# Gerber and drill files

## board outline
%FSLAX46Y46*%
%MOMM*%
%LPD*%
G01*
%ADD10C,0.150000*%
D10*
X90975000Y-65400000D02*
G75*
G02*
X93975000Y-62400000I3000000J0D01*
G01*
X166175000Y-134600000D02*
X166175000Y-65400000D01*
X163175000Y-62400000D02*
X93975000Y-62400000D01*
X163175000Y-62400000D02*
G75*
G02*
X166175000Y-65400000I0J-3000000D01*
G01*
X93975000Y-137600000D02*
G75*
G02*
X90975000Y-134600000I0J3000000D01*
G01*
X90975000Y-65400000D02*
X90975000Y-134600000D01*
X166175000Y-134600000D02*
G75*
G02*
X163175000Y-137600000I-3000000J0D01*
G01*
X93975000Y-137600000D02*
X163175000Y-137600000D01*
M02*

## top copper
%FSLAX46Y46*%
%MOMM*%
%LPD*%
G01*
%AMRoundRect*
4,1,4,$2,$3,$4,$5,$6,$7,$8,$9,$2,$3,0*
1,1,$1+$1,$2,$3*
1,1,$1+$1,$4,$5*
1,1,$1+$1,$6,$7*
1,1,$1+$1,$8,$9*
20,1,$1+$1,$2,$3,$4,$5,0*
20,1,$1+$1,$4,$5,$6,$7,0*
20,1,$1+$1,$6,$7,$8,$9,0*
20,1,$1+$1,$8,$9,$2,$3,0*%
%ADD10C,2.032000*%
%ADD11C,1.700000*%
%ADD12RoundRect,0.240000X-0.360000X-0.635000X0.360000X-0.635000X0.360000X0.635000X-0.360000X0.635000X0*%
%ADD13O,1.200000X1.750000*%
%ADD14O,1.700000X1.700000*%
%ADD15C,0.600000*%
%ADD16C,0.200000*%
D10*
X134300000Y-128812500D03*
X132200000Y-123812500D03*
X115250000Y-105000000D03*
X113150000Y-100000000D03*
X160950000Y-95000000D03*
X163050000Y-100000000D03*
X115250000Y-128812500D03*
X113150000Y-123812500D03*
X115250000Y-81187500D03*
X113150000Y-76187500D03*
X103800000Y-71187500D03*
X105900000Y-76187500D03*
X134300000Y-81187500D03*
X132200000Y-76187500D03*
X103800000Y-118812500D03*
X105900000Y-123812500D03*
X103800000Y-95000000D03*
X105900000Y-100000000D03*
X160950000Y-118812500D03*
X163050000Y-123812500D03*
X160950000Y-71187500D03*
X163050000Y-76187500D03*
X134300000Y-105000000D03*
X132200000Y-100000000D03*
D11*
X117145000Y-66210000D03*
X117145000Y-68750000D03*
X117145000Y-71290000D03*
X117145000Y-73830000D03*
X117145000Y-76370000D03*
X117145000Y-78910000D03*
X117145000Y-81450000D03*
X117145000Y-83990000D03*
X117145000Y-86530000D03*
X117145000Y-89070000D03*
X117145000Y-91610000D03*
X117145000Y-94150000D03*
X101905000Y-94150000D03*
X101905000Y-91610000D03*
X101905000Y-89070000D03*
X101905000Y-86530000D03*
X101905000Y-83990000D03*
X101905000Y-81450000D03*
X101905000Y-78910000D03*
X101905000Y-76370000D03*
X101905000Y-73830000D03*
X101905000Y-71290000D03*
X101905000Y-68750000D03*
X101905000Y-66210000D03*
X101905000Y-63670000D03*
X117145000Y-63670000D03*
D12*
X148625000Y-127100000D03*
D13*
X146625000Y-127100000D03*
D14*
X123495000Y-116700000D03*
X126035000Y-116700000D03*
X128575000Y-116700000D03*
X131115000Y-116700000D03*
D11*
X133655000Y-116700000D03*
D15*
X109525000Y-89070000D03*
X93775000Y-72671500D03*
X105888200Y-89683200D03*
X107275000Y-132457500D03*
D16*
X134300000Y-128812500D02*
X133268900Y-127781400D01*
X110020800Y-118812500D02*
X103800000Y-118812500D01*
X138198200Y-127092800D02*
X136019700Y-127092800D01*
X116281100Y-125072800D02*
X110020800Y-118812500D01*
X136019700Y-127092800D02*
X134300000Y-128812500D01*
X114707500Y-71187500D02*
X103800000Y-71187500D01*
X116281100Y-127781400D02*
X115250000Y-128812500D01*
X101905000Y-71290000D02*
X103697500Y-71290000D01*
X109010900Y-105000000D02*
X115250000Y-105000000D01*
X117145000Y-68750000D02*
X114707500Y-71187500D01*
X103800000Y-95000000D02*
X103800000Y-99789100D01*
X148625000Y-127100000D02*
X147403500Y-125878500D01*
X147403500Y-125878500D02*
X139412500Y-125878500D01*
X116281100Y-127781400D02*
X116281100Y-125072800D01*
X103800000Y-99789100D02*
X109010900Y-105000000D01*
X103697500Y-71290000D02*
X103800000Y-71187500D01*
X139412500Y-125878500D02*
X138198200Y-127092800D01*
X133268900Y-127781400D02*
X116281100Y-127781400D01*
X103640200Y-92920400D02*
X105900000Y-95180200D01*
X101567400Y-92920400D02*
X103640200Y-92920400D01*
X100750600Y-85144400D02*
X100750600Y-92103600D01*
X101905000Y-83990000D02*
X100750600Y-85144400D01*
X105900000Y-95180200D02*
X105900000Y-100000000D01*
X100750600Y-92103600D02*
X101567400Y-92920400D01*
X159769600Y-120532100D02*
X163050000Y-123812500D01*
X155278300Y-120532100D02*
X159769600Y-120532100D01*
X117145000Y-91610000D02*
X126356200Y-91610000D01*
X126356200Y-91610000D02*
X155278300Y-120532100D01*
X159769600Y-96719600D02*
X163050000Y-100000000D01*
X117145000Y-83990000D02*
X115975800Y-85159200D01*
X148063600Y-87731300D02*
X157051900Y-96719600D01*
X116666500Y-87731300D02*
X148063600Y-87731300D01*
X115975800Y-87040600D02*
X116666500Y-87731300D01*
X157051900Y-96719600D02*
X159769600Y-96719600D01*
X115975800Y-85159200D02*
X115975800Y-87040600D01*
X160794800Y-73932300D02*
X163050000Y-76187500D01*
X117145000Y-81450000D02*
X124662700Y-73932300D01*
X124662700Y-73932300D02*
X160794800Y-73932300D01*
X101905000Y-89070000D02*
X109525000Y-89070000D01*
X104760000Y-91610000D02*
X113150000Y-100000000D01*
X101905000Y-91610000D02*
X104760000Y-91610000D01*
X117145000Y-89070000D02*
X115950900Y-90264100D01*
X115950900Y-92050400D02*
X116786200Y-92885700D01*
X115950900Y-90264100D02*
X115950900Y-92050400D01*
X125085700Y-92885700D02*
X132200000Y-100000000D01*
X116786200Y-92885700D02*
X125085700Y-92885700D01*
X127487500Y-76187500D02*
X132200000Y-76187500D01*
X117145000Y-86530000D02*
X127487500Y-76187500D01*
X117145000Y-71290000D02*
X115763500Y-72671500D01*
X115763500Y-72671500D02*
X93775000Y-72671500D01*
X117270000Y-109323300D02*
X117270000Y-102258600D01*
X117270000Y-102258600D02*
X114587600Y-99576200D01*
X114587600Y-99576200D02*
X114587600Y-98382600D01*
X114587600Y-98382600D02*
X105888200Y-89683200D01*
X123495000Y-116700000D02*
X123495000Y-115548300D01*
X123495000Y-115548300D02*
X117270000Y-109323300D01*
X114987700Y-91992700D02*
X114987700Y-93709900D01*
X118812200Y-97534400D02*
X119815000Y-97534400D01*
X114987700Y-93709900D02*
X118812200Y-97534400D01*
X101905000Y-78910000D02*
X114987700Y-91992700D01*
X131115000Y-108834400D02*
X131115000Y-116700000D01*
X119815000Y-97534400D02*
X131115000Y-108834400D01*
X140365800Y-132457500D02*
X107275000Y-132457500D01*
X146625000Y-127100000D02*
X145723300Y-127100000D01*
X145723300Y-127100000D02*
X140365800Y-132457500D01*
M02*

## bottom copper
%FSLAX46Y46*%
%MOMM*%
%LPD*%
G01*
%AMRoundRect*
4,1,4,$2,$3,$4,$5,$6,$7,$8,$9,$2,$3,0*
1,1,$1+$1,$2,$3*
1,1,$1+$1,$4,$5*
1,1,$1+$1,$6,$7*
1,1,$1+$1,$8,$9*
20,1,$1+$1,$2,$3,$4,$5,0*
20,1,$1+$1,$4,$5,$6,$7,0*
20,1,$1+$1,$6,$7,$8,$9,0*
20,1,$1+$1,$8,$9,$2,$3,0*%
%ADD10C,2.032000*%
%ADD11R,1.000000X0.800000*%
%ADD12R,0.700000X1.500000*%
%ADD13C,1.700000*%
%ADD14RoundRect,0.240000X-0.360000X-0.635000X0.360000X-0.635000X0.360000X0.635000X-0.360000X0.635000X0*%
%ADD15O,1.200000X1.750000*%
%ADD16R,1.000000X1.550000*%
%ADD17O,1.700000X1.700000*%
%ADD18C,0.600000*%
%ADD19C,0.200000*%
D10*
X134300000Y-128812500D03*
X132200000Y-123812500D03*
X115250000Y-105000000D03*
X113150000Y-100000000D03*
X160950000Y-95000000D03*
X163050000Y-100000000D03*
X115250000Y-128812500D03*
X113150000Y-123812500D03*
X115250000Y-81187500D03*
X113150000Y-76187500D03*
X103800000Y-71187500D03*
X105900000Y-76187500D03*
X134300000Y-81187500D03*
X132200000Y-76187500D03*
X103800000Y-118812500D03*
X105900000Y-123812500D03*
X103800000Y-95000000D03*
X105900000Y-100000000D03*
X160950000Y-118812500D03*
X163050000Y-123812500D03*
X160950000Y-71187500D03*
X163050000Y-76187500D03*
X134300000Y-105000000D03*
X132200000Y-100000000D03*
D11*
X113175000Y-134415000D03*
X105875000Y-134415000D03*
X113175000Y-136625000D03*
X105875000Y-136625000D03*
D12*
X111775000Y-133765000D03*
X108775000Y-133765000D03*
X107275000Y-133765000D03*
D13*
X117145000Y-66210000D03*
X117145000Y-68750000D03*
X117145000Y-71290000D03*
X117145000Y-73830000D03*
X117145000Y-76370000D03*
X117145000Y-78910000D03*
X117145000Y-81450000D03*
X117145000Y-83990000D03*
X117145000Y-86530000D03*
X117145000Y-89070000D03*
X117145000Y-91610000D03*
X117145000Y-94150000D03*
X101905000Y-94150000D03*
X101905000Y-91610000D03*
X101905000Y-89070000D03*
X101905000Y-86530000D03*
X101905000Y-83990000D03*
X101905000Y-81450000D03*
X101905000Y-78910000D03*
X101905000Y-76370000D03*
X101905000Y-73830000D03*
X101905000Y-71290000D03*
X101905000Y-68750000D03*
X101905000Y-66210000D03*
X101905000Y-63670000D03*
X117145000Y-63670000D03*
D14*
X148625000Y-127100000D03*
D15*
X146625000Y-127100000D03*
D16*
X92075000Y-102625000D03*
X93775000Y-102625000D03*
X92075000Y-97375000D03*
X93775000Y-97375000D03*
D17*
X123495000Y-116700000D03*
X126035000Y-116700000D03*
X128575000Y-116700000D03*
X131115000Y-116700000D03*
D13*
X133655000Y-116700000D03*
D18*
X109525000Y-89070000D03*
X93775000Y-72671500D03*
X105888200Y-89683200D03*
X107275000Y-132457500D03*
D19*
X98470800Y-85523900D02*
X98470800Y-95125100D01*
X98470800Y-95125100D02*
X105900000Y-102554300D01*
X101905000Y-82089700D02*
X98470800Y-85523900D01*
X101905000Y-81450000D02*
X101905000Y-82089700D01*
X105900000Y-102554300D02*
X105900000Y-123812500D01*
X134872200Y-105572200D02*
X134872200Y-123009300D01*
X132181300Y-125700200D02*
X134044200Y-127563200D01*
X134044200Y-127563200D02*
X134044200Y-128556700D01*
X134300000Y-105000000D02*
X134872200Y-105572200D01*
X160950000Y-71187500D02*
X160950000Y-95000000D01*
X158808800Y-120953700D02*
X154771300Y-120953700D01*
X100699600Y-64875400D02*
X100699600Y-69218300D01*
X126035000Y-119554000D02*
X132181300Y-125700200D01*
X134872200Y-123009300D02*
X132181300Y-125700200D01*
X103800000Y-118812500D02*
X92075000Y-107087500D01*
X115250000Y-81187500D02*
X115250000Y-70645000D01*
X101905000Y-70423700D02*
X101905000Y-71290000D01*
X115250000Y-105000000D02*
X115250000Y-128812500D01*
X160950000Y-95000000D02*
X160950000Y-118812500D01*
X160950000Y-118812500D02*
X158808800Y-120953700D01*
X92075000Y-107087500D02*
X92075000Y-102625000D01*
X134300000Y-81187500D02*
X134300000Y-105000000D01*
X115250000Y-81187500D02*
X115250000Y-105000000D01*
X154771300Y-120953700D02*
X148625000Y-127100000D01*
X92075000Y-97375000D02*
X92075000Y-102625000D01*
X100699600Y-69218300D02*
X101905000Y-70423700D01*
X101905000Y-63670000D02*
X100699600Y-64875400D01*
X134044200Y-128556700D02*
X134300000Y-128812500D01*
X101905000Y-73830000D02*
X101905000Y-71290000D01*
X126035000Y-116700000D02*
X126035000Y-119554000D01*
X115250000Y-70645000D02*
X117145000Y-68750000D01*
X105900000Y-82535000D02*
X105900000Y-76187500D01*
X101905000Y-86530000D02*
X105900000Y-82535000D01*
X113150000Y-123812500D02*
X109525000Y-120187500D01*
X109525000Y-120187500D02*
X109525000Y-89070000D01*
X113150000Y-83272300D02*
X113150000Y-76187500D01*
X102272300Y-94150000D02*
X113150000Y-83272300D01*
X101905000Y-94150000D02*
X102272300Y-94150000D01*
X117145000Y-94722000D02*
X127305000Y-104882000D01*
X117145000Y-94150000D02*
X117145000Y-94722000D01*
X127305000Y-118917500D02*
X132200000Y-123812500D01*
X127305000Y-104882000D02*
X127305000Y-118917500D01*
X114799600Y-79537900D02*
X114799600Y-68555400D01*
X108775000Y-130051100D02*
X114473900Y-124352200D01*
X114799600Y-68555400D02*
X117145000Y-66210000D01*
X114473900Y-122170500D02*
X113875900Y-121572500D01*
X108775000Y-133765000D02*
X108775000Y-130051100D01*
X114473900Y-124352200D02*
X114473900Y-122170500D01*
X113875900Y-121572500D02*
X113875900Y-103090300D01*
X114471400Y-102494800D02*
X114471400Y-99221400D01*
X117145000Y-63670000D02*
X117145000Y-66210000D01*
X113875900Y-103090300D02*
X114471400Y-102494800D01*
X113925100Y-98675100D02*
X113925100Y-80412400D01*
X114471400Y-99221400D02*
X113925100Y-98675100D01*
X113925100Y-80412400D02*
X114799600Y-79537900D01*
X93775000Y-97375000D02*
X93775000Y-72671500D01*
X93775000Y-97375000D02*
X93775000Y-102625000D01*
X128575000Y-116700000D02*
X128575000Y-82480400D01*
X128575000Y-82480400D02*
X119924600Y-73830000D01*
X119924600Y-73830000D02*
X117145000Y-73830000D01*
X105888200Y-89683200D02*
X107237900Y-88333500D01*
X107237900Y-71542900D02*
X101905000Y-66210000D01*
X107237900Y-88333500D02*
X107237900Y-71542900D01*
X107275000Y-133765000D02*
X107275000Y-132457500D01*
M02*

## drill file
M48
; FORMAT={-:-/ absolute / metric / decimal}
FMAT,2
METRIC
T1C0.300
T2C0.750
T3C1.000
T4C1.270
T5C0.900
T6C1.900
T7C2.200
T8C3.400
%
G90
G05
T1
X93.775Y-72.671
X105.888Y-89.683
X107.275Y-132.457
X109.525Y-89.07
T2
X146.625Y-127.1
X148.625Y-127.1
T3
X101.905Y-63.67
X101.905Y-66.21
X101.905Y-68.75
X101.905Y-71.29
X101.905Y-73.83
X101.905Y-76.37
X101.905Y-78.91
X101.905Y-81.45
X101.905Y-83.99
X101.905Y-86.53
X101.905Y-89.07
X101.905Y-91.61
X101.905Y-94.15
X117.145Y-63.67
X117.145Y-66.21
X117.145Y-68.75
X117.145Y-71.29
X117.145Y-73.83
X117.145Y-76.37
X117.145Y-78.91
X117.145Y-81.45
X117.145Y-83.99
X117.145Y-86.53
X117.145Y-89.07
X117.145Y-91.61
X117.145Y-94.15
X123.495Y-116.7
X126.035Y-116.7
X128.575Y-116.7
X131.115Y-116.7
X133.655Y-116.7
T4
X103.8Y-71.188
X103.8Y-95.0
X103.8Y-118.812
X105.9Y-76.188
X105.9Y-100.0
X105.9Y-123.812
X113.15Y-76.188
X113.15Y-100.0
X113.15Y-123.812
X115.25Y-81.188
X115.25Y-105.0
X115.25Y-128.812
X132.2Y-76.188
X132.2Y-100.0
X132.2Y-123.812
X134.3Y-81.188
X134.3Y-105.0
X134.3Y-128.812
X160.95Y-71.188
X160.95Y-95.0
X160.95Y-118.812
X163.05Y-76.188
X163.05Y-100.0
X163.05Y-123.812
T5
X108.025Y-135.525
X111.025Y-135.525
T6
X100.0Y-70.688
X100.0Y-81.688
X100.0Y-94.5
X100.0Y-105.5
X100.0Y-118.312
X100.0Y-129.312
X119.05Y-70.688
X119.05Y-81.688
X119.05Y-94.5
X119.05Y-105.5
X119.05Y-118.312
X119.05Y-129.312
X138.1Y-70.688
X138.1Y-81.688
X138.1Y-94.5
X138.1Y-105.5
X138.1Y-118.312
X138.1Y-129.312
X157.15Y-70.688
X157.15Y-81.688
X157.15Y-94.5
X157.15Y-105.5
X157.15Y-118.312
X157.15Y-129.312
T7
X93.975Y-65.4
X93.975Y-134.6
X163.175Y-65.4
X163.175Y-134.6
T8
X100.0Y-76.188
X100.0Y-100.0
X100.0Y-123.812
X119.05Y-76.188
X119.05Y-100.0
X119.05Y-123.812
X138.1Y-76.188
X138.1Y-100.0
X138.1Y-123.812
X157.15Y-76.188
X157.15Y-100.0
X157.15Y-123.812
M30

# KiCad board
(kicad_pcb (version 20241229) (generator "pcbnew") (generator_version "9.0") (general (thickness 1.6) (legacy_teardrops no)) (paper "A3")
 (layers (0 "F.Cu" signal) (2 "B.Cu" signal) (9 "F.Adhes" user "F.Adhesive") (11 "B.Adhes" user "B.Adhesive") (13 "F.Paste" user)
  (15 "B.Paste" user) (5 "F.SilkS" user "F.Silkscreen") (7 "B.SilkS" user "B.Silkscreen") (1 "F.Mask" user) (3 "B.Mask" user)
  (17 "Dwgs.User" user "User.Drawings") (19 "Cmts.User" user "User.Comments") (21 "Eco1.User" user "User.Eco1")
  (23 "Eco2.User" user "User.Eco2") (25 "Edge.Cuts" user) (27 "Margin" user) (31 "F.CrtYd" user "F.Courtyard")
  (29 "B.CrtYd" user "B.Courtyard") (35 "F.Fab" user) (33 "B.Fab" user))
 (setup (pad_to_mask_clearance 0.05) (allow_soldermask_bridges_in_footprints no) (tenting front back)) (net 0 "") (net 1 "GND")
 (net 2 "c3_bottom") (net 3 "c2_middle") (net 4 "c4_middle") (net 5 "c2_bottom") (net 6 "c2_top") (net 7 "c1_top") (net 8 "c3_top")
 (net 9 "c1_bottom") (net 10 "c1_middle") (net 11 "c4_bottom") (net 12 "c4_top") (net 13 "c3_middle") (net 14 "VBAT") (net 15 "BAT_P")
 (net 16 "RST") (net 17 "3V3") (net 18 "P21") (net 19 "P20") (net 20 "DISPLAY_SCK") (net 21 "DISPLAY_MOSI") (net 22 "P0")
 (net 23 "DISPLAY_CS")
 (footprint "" (layer "F.Cu") (at 128.574999 100)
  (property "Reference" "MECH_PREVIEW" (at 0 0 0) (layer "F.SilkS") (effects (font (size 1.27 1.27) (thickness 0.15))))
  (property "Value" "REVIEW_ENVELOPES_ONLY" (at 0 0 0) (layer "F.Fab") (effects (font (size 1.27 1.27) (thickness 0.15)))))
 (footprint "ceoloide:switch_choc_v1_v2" (layer "F.Cu") (at 138.1 123.8125 90)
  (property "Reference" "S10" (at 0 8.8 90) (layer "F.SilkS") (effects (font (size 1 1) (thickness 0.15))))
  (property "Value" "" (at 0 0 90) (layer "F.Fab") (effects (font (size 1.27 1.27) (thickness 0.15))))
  (pad "" np_thru_hole circle (at -5.5 0 90) (size 1.9 1.9) (drill 1.9) (layers "*.Cu" "*.Mask"))
  (pad "" np_thru_hole circle (at 0 0 90) (size 3.4 3.4) (drill 3.4) (layers "*.Cu" "*.Mask"))
  (pad "" np_thru_hole circle (at 5.5 0 90) (size 1.9 1.9) (drill 1.9) (layers "*.Cu" "*.Mask"))
  (pad "1" thru_hole circle (at -5 -3.8 285) (size 2.032 2.032) (drill 1.27) (layers "*.Cu" "*.Mask") (remove_unused_layers no)
   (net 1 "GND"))
  (pad "2" thru_hole circle (at 0 -5.9 285) (size 2.032 2.032) (drill 1.27) (layers "*.Cu" "*.Mask") (remove_unused_layers no)
   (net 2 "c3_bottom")))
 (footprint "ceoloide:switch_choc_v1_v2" (layer "F.Cu") (at 119.05 100 90)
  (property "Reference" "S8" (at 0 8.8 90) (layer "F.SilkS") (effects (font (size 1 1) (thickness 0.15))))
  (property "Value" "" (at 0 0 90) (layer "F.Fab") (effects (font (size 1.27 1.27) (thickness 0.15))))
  (pad "" np_thru_hole circle (at -5.5 0 90) (size 1.9 1.9) (drill 1.9) (layers "*.Cu" "*.Mask"))
  (pad "" np_thru_hole circle (at 0 0 90) (size 3.4 3.4) (drill 3.4) (layers "*.Cu" "*.Mask"))
  (pad "" np_thru_hole circle (at 5.5 0 90) (size 1.9 1.9) (drill 1.9) (layers "*.Cu" "*.Mask"))
  (pad "1" thru_hole circle (at -5 -3.8 285) (size 2.032 2.032) (drill 1.27) (layers "*.Cu" "*.Mask") (remove_unused_layers no)
   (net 1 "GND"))
  (pad "2" thru_hole circle (at 0 -5.9 285) (size 2.032 2.032) (drill 1.27) (layers "*.Cu" "*.Mask") (remove_unused_layers no)
   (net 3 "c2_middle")))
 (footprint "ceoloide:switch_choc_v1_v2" (layer "F.Cu") (at 157.15 100 -90)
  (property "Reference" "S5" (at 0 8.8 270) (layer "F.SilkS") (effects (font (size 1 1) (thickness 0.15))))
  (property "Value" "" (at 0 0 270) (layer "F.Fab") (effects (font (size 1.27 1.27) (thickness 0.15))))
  (pad "" np_thru_hole circle (at -5.5 0 270) (size 1.9 1.9) (drill 1.9) (layers "*.Cu" "*.Mask"))
  (pad "" np_thru_hole circle (at 0 0 270) (size 3.4 3.4) (drill 3.4) (layers "*.Cu" "*.Mask"))
  (pad "" np_thru_hole circle (at 5.5 0 270) (size 1.9 1.9) (drill 1.9) (layers "*.Cu" "*.Mask"))
  (pad "1" thru_hole circle (at -5 -3.8 105) (size 2.032 2.032) (drill 1.27) (layers "*.Cu" "*.Mask") (remove_unused_layers no)
   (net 1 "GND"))
  (pad "2" thru_hole circle (at 0 -5.9 105) (size 2.032 2.032) (drill 1.27) (layers "*.Cu" "*.Mask") (remove_unused_layers no)
   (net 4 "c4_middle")))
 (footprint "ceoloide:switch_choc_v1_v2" (layer "F.Cu") (at 119.05 123.8125 90)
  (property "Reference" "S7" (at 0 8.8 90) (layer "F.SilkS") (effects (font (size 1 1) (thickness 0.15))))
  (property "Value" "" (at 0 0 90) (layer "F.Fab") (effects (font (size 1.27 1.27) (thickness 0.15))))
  (pad "" np_thru_hole circle (at -5.5 0 90) (size 1.9 1.9) (drill 1.9) (layers "*.Cu" "*.Mask"))
  (pad "" np_thru_hole circle (at 0 0 90) (size 3.4 3.4) (drill 3.4) (layers "*.Cu" "*.Mask"))
  (pad "" np_thru_hole circle (at 5.5 0 90) (size 1.9 1.9) (drill 1.9) (layers "*.Cu" "*.Mask"))
  (pad "1" thru_hole circle (at -5 -3.8 285) (size 2.032 2.032) (drill 1.27) (layers "*.Cu" "*.Mask") (remove_unused_layers no)
   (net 1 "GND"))
  (pad "2" thru_hole circle (at 0 -5.9 285) (size 2.032 2.032) (drill 1.27) (layers "*.Cu" "*.Mask") (remove_unused_layers no)
   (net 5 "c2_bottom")))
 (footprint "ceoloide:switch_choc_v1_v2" (layer "F.Cu") (at 119.05 76.1875 90)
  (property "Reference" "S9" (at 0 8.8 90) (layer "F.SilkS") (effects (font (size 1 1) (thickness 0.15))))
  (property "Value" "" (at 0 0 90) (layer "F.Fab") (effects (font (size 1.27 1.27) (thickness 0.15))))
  (pad "" np_thru_hole circle (at -5.5 0 90) (size 1.9 1.9) (drill 1.9) (layers "*.Cu" "*.Mask"))
  (pad "" np_thru_hole circle (at 0 0 90) (size 3.4 3.4) (drill 3.4) (layers "*.Cu" "*.Mask"))
  (pad "" np_thru_hole circle (at 5.5 0 90) (size 1.9 1.9) (drill 1.9) (layers "*.Cu" "*.Mask"))
  (pad "1" thru_hole circle (at -5 -3.8 285) (size 2.032 2.032) (drill 1.27) (layers "*.Cu" "*.Mask") (remove_unused_layers no)
   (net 1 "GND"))
  (pad "2" thru_hole circle (at 0 -5.9 285) (size 2.032 2.032) (drill 1.27) (layers "*.Cu" "*.Mask") (remove_unused_layers no)
   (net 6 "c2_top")))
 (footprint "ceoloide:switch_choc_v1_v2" (layer "F.Cu") (at 100 76.1875 -90)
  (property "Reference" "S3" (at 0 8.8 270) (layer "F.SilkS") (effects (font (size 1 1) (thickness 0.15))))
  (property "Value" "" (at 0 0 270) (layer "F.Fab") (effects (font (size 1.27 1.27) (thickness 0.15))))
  (pad "" np_thru_hole circle (at -5.5 0 270) (size 1.9 1.9) (drill 1.9) (layers "*.Cu" "*.Mask"))
  (pad "" np_thru_hole circle (at 0 0 270) (size 3.4 3.4) (drill 3.4) (layers "*.Cu" "*.Mask"))
  (pad "" np_thru_hole circle (at 5.5 0 270) (size 1.9 1.9) (drill 1.9) (layers "*.Cu" "*.Mask"))
  (pad "1" thru_hole circle (at -5 -3.8 105) (size 2.032 2.032) (drill 1.27) (layers "*.Cu" "*.Mask") (remove_unused_layers no)
   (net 1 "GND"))
  (pad "2" thru_hole circle (at 0 -5.9 105) (size 2.032 2.032) (drill 1.27) (layers "*.Cu" "*.Mask") (remove_unused_layers no)
   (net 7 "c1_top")))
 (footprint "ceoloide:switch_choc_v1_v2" (layer "F.Cu") (at 138.1 76.1875 90)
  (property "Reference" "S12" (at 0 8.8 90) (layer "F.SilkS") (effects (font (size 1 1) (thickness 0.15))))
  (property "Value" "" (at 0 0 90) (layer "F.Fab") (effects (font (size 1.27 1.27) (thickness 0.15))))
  (pad "" np_thru_hole circle (at -5.5 0 90) (size 1.9 1.9) (drill 1.9) (layers "*.Cu" "*.Mask"))
  (pad "" np_thru_hole circle (at 0 0 90) (size 3.4 3.4) (drill 3.4) (layers "*.Cu" "*.Mask"))
  (pad "" np_thru_hole circle (at 5.5 0 90) (size 1.9 1.9) (drill 1.9) (layers "*.Cu" "*.Mask"))
  (pad "1" thru_hole circle (at -5 -3.8 285) (size 2.032 2.032) (drill 1.27) (layers "*.Cu" "*.Mask") (remove_unused_layers no)
   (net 1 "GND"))
  (pad "2" thru_hole circle (at 0 -5.9 285) (size 2.032 2.032) (drill 1.27) (layers "*.Cu" "*.Mask") (remove_unused_layers no)
   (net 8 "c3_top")))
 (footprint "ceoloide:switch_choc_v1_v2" (layer "F.Cu") (at 100 123.8125 -90)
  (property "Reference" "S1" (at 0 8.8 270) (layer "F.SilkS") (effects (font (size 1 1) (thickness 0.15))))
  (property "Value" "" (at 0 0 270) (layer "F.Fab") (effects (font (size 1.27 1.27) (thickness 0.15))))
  (pad "" np_thru_hole circle (at -5.5 0 270) (size 1.9 1.9) (drill 1.9) (layers "*.Cu" "*.Mask"))
  (pad "" np_thru_hole circle (at 0 0 270) (size 3.4 3.4) (drill 3.4) (layers "*.Cu" "*.Mask"))
  (pad "" np_thru_hole circle (at 5.5 0 270) (size 1.9 1.9) (drill 1.9) (layers "*.Cu" "*.Mask"))
  (pad "1" thru_hole circle (at -5 -3.8 105) (size 2.032 2.032) (drill 1.27) (layers "*.Cu" "*.Mask") (remove_unused_layers no)
   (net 1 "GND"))
  (pad "2" thru_hole circle (at 0 -5.9 105) (size 2.032 2.032) (drill 1.27) (layers "*.Cu" "*.Mask") (remove_unused_layers no)
   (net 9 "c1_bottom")))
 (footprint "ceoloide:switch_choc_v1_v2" (layer "F.Cu") (at 100 100 -90)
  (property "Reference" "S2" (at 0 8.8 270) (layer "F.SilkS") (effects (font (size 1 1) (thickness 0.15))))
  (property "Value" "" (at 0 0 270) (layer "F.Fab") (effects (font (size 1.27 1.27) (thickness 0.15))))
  (pad "" np_thru_hole circle (at -5.5 0 270) (size 1.9 1.9) (drill 1.9) (layers "*.Cu" "*.Mask"))
  (pad "" np_thru_hole circle (at 0 0 270) (size 3.4 3.4) (drill 3.4) (layers "*.Cu" "*.Mask"))
  (pad "" np_thru_hole circle (at 5.5 0 270) (size 1.9 1.9) (drill 1.9) (layers "*.Cu" "*.Mask"))
  (pad "1" thru_hole circle (at -5 -3.8 105) (size 2.032 2.032) (drill 1.27) (layers "*.Cu" "*.Mask") (remove_unused_layers no)
   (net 1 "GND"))
  (pad "2" thru_hole circle (at 0 -5.9 105) (size 2.032 2.032) (drill 1.27) (layers "*.Cu" "*.Mask") (remove_unused_layers no)
   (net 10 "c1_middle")))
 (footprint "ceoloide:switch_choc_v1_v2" (layer "F.Cu") (at 157.15 123.8125 -90)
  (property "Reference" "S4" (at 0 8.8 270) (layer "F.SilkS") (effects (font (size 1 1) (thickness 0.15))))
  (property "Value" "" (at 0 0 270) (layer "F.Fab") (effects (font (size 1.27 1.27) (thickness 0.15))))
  (pad "" np_thru_hole circle (at -5.5 0 270) (size 1.9 1.9) (drill 1.9) (layers "*.Cu" "*.Mask"))
  (pad "" np_thru_hole circle (at 0 0 270) (size 3.4 3.4) (drill 3.4) (layers "*.Cu" "*.Mask"))
  (pad "" np_thru_hole circle (at 5.5 0 270) (size 1.9 1.9) (drill 1.9) (layers "*.Cu" "*.Mask"))
  (pad "1" thru_hole circle (at -5 -3.8 105) (size 2.032 2.032) (drill 1.27) (layers "*.Cu" "*.Mask") (remove_unused_layers no)
   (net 1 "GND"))
  (pad "2" thru_hole circle (at 0 -5.9 105) (size 2.032 2.032) (drill 1.27) (layers "*.Cu" "*.Mask") (remove_unused_layers no)
   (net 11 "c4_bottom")))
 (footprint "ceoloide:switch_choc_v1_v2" (layer "F.Cu") (at 157.15 76.1875 -90)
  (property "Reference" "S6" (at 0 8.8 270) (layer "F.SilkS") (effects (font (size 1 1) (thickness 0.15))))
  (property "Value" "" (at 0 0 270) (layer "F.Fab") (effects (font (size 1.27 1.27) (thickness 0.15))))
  (pad "" np_thru_hole circle (at -5.5 0 270) (size 1.9 1.9) (drill 1.9) (layers "*.Cu" "*.Mask"))
  (pad "" np_thru_hole circle (at 0 0 270) (size 3.4 3.4) (drill 3.4) (layers "*.Cu" "*.Mask"))
  (pad "" np_thru_hole circle (at 5.5 0 270) (size 1.9 1.9) (drill 1.9) (layers "*.Cu" "*.Mask"))
  (pad "1" thru_hole circle (at -5 -3.8 105) (size 2.032 2.032) (drill 1.27) (layers "*.Cu" "*.Mask") (remove_unused_layers no)
   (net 1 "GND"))
  (pad "2" thru_hole circle (at 0 -5.9 105) (size 2.032 2.032) (drill 1.27) (layers "*.Cu" "*.Mask") (remove_unused_layers no)
   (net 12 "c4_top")))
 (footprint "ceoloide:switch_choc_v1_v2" (layer "F.Cu") (at 138.1 100 90)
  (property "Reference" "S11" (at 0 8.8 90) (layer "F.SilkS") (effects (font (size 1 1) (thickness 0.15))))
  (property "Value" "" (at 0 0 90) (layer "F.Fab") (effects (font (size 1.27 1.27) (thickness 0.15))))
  (pad "" np_thru_hole circle (at -5.5 0 90) (size 1.9 1.9) (drill 1.9) (layers "*.Cu" "*.Mask"))
  (pad "" np_thru_hole circle (at 0 0 90) (size 3.4 3.4) (drill 3.4) (layers "*.Cu" "*.Mask"))
  (pad "" np_thru_hole circle (at 5.5 0 90) (size 1.9 1.9) (drill 1.9) (layers "*.Cu" "*.Mask"))
  (pad "1" thru_hole circle (at -5 -3.8 285) (size 2.032 2.032) (drill 1.27) (layers "*.Cu" "*.Mask") (remove_unused_layers no)
   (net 1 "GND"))
  (pad "2" thru_hole circle (at 0 -5.9 285) (size 2.032 2.032) (drill 1.27) (layers "*.Cu" "*.Mask") (remove_unused_layers no)
   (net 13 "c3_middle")))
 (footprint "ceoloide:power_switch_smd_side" (layer "B.Cu") (at 109.525 135.5 -90)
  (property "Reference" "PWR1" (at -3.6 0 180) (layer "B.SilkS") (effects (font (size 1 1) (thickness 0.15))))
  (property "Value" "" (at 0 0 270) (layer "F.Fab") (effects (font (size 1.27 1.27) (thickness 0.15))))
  (pad "" smd rect (at -1.085 -3.65 180) (size 1 0.8) (layers "B.Cu" "B.Mask" "B.Paste"))
  (pad "" smd rect (at -1.085 3.65 180) (size 1 0.8) (layers "B.Cu" "B.Mask" "B.Paste"))
  (pad "" np_thru_hole circle (at 0.025 -1.5) (size 0.9 0.9) (drill 0.9) (layers "*.Cu" "*.Mask"))
  (pad "" np_thru_hole circle (at 0.025 1.5) (size 0.9 0.9) (drill 0.9) (layers "*.Cu" "*.Mask"))
  (pad "" smd rect (at 1.125 -3.65 180) (size 1 0.8) (layers "B.Cu" "B.Mask" "B.Paste"))
  (pad "" smd rect (at 1.125 3.65 180) (size 1 0.8) (layers "B.Cu" "B.Mask" "B.Paste"))
  (pad "1" smd rect (at -1.735 -2.25 180) (size 0.7 1.5) (layers "B.Cu" "B.Mask" "B.Paste"))
  (pad "2" smd rect (at -1.735 0.75 180) (size 0.7 1.5) (layers "B.Cu" "B.Mask" "B.Paste") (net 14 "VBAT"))
  (pad "3" smd rect (at -1.735 2.25 180) (size 0.7 1.5) (layers "B.Cu" "B.Mask" "B.Paste") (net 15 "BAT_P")))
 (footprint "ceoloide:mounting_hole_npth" (layer "B.Cu") (at 93.975 134.6)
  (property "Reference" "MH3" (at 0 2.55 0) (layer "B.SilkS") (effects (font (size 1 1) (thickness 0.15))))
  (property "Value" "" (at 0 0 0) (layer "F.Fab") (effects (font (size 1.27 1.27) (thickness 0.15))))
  (pad "" np_thru_hole circle (at 0 0) (size 2.2 2.2) (drill 2.2) (layers "*.Cu" "*.Mask")))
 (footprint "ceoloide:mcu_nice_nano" (layer "B.Cu") (at 109.525 78.91)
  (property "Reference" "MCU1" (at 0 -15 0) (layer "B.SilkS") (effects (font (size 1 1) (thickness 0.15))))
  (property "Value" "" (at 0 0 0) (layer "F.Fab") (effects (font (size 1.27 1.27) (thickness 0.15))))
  (pad "1" thru_hole circle (at 7.62 -12.7) (size 1.7 1.7) (drill 1) (layers "*.Cu" "*.Mask") (remove_unused_layers no) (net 14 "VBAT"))
  (pad "2" thru_hole circle (at 7.62 -10.16) (size 1.7 1.7) (drill 1) (layers "*.Cu" "*.Mask") (remove_unused_layers no) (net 1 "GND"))
  (pad "3" thru_hole circle (at 7.62 -7.62) (size 1.7 1.7) (drill 1) (layers "*.Cu" "*.Mask") (remove_unused_layers no) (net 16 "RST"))
  (pad "4" thru_hole circle (at 7.62 -5.08) (size 1.7 1.7) (drill 1) (layers "*.Cu" "*.Mask") (remove_unused_layers no) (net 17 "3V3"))
  (pad "5" thru_hole circle (at 7.62 -2.54) (size 1.7 1.7) (drill 1) (layers "*.Cu" "*.Mask") (remove_unused_layers no) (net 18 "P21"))
  (pad "6" thru_hole circle (at 7.62 0) (size 1.7 1.7) (drill 1) (layers "*.Cu" "*.Mask") (remove_unused_layers no) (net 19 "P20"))
  (pad "7" thru_hole circle (at 7.62 2.54) (size 1.7 1.7) (drill 1) (layers "*.Cu" "*.Mask") (remove_unused_layers no) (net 12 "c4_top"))
  (pad "8" thru_hole circle (at 7.62 5.08) (size 1.7 1.7) (drill 1) (layers "*.Cu" "*.Mask") (remove_unused_layers no) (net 4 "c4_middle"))
  (pad "9" thru_hole circle (at 7.62 7.62) (size 1.7 1.7) (drill 1) (layers "*.Cu" "*.Mask") (remove_unused_layers no) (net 8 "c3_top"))
  (pad "10" thru_hole circle (at 7.62 10.16) (size 1.7 1.7) (drill 1) (layers "*.Cu" "*.Mask") (remove_unused_layers no)
   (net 13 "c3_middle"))
  (pad "11" thru_hole circle (at 7.62 12.7) (size 1.7 1.7) (drill 1) (layers "*.Cu" "*.Mask") (remove_unused_layers no) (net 11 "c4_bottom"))
  (pad "12" thru_hole circle (at 7.62 15.24) (size 1.7 1.7) (drill 1) (layers "*.Cu" "*.Mask") (remove_unused_layers no) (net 2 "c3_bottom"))
  (pad "13" thru_hole circle (at -7.62 15.24) (size 1.7 1.7) (drill 1) (layers "*.Cu" "*.Mask") (remove_unused_layers no) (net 6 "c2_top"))
  (pad "14" thru_hole circle (at -7.62 12.7) (size 1.7 1.7) (drill 1) (layers "*.Cu" "*.Mask") (remove_unused_layers no) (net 3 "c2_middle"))
  (pad "15" thru_hole circle (at -7.62 10.16) (size 1.7 1.7) (drill 1) (layers "*.Cu" "*.Mask") (remove_unused_layers no)
   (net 5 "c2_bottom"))
  (pad "16" thru_hole circle (at -7.62 7.62) (size 1.7 1.7) (drill 1) (layers "*.Cu" "*.Mask") (remove_unused_layers no) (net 7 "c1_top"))
  (pad "17" thru_hole circle (at -7.62 5.08) (size 1.7 1.7) (drill 1) (layers "*.Cu" "*.Mask") (remove_unused_layers no)
   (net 10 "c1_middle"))
  (pad "18" thru_hole circle (at -7.62 2.54) (size 1.7 1.7) (drill 1) (layers "*.Cu" "*.Mask") (remove_unused_layers no) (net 9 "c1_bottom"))
  (pad "19" thru_hole circle (at -7.62 0) (size 1.7 1.7) (drill 1) (layers "*.Cu" "*.Mask") (remove_unused_layers no) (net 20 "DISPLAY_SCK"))
  (pad "20" thru_hole circle (at -7.62 -2.54) (size 1.7 1.7) (drill 1) (layers "*.Cu" "*.Mask") (remove_unused_layers no)
   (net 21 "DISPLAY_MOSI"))
  (pad "21" thru_hole circle (at -7.62 -5.08) (size 1.7 1.7) (drill 1) (layers "*.Cu" "*.Mask") (remove_unused_layers no) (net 1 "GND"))
  (pad "22" thru_hole circle (at -7.62 -7.62) (size 1.7 1.7) (drill 1) (layers "*.Cu" "*.Mask") (remove_unused_layers no) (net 1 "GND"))
  (pad "23" thru_hole circle (at -7.62 -10.16) (size 1.7 1.7) (drill 1) (layers "*.Cu" "*.Mask") (remove_unused_layers no) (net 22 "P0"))
  (pad "24" thru_hole circle (at -7.62 -12.7) (size 1.7 1.7) (drill 1) (layers "*.Cu" "*.Mask") (remove_unused_layers no)
   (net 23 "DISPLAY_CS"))
  (pad "25" thru_hole circle (at -7.62 -15.24) (size 1.7 1.7) (drill 1) (layers "*.Cu" "*.Mask") (remove_unused_layers no) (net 1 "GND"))
  (pad "26" thru_hole circle (at 7.62 -15.24) (size 1.7 1.7) (drill 1) (layers "*.Cu" "*.Mask") (remove_unused_layers no) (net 14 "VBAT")))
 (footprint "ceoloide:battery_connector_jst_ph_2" (layer "B.Cu") (at 147.625 127.1)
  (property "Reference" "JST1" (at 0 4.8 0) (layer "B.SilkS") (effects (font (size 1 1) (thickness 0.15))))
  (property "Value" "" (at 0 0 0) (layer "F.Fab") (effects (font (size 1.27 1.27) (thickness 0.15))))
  (pad "1" thru_hole roundrect (at 1 0) (size 1.2 1.75) (drill 0.75) (layers "*.Cu" "*.Mask") (remove_unused_layers no)
   (roundrect_rratio 0.2) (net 1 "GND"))
  (pad "2" thru_hole oval (at -1 0) (size 1.2 1.75) (drill 0.75) (layers "*.Cu" "*.Mask") (remove_unused_layers no) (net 15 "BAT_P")))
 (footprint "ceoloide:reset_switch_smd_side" (layer "B.Cu") (at 92.925 100 90)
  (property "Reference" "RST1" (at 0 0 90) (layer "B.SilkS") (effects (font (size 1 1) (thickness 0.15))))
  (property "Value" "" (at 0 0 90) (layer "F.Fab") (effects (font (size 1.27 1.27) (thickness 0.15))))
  (pad "1" smd rect (at -2.625 -0.85 270) (size 1.55 1) (layers "B.Cu" "B.Mask" "B.Paste") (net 1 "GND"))
  (pad "2" smd rect (at -2.625 0.85 270) (size 1.55 1) (layers "B.Cu" "B.Mask" "B.Paste") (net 16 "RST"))
  (pad "3" smd rect (at 2.625 -0.85 270) (size 1.55 1) (layers "B.Cu" "B.Mask" "B.Paste") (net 1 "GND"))
  (pad "4" smd rect (at 2.625 0.85 270) (size 1.55 1) (layers "B.Cu" "B.Mask" "B.Paste") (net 16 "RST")))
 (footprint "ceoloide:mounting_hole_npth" (layer "B.Cu") (at 163.175 65.4)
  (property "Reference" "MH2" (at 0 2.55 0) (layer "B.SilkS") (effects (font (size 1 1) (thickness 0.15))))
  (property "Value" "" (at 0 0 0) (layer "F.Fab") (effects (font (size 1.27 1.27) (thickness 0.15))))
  (pad "" np_thru_hole circle (at 0 0) (size 2.2 2.2) (drill 2.2) (layers "*.Cu" "*.Mask")))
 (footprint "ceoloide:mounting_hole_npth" (layer "B.Cu") (at 163.175 134.6)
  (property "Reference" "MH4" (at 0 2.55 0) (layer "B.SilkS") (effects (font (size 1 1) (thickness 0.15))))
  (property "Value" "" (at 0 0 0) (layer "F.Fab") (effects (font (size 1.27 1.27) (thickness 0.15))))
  (pad "" np_thru_hole circle (at 0 0) (size 2.2 2.2) (drill 2.2) (layers "*.Cu" "*.Mask")))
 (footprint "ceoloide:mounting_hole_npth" (layer "B.Cu") (at 93.975 65.4)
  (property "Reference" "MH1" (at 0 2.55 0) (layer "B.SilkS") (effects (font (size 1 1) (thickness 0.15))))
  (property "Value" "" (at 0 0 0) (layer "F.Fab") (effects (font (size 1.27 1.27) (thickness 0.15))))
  (pad "" np_thru_hole circle (at 0 0) (size 2.2 2.2) (drill 2.2) (layers "*.Cu" "*.Mask")))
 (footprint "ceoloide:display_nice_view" (layer "B.Cu") (at 128.575 100)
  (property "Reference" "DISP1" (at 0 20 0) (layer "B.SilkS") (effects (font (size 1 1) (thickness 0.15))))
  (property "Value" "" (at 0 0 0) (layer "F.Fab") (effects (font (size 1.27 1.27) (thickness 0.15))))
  (pad "1" thru_hole oval (at -5.08 16.7 270) (size 1.7 1.7) (drill 1) (layers "*.Cu" "*.Mask") (remove_unused_layers no)
   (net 23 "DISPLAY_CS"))
  (pad "2" thru_hole oval (at -2.54 16.7 270) (size 1.7 1.7) (drill 1) (layers "*.Cu" "*.Mask") (remove_unused_layers no) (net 1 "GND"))
  (pad "3" thru_hole oval (at 0 16.7 270) (size 1.7 1.7) (drill 1) (layers "*.Cu" "*.Mask") (remove_unused_layers no) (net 17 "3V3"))
  (pad "4" thru_hole oval (at 2.54 16.7 270) (size 1.7 1.7) (drill 1) (layers "*.Cu" "*.Mask") (remove_unused_layers no)
   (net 20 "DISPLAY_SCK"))
  (pad "5" thru_hole circle (at 5.08 16.7 270) (size 1.7 1.7) (drill 1) (layers "*.Cu" "*.Mask") (remove_unused_layers no)
   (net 21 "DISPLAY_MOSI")))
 (gr_arc (start 90.975 65.4) (mid 91.85368 63.27868) (end 93.975 62.4) (stroke (width 0.15) (type default)) (layer "Edge.Cuts"))
 (gr_line (start 166.175 134.6) (end 166.175 65.4) (stroke (width 0.15) (type default)) (layer "Edge.Cuts"))
 (gr_line (start 163.175 62.4) (end 93.975 62.4) (stroke (width 0.15) (type default)) (layer "Edge.Cuts"))
 (gr_arc (start 163.175 62.4) (mid 165.29632 63.27868) (end 166.175 65.4) (stroke (width 0.15) (type default)) (layer "Edge.Cuts"))
 (gr_arc (start 93.975 137.6) (mid 91.85368 136.72132) (end 90.975 134.6) (stroke (width 0.15) (type default)) (layer "Edge.Cuts"))
 (gr_line (start 90.975 65.4) (end 90.975 134.6) (stroke (width 0.15) (type default)) (layer "Edge.Cuts"))
 (gr_arc (start 166.175 134.6) (mid 165.29632 136.72132) (end 163.175 137.6) (stroke (width 0.15) (type default)) (layer "Edge.Cuts"))
 (gr_line (start 93.975 137.6) (end 163.175 137.6) (stroke (width 0.15) (type default)) (layer "Edge.Cuts"))
 (segment (start 98.4708 85.5239) (end 98.4708 95.1251) (width 0.2) (layer "B.Cu") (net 9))
 (segment (start 98.4708 95.1251) (end 105.9 102.5543) (width 0.2) (layer "B.Cu") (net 9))
 (segment (start 101.905 82.0897) (end 98.4708 85.5239) (width 0.2) (layer "B.Cu") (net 9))
 (segment (start 101.905 81.45) (end 101.905 82.0897) (width 0.2) (layer "B.Cu") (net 9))
 (segment (start 105.9 102.5543) (end 105.9 123.8125) (width 0.2) (layer "B.Cu") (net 9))
 (segment (start 134.3 128.8125) (end 133.2689 127.7814) (width 0.2) (layer "F.Cu") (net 1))
 (segment (start 110.0208 118.8125) (end 103.8 118.8125) (width 0.2) (layer "F.Cu") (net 1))
 (segment (start 138.1982 127.0928) (end 136.0197 127.0928) (width 0.2) (layer "F.Cu") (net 1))
 (segment (start 116.2811 125.0728) (end 110.0208 118.8125) (width 0.2) (layer "F.Cu") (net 1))
 (segment (start 136.0197 127.0928) (end 134.3 128.8125) (width 0.2) (layer "F.Cu") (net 1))
 (segment (start 114.7075 71.1875) (end 103.8 71.1875) (width 0.2) (layer "F.Cu") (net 1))
 (segment (start 116.2811 127.7814) (end 115.25 128.8125) (width 0.2) (layer "F.Cu") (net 1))
 (segment (start 101.905 71.29) (end 103.6975 71.29) (width 0.2) (layer "F.Cu") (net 1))
 (segment (start 109.0109 105) (end 115.25 105) (width 0.2) (layer "F.Cu") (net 1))
 (segment (start 117.145 68.75) (end 114.7075 71.1875) (width 0.2) (layer "F.Cu") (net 1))
 (segment (start 103.8 95) (end 103.8 99.7891) (width 0.2) (layer "F.Cu") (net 1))
 (segment (start 148.625 127.1) (end 147.4035 125.8785) (width 0.2) (layer "F.Cu") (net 1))
 (segment (start 147.4035 125.8785) (end 139.4125 125.8785) (width 0.2) (layer "F.Cu") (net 1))
 (segment (start 116.2811 127.7814) (end 116.2811 125.0728) (width 0.2) (layer "F.Cu") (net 1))
 (segment (start 103.8 99.7891) (end 109.0109 105) (width 0.2) (layer "F.Cu") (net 1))
 (segment (start 103.6975 71.29) (end 103.8 71.1875) (width 0.2) (layer "F.Cu") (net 1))
 (segment (start 139.4125 125.8785) (end 138.1982 127.0928) (width 0.2) (layer "F.Cu") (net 1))
 (segment (start 133.2689 127.7814) (end 116.2811 127.7814) (width 0.2) (layer "F.Cu") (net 1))
 (segment (start 134.8722 105.5722) (end 134.8722 123.0093) (width 0.2) (layer "B.Cu") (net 1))
 (segment (start 132.1813 125.7002) (end 134.0442 127.5632) (width 0.2) (layer "B.Cu") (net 1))
 (segment (start 134.0442 127.5632) (end 134.0442 128.5567) (width 0.2) (layer "B.Cu") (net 1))
 (segment (start 134.3 105) (end 134.8722 105.5722) (width 0.2) (layer "B.Cu") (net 1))
 (segment (start 160.95 71.1875) (end 160.95 95) (width 0.2) (layer "B.Cu") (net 1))
 (segment (start 158.8088 120.9537) (end 154.7713 120.9537) (width 0.2) (layer "B.Cu") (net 1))
 (segment (start 100.6996 64.8754) (end 100.6996 69.2183) (width 0.2) (layer "B.Cu") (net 1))
 (segment (start 126.035 119.554) (end 132.1813 125.7002) (width 0.2) (layer "B.Cu") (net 1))
 (segment (start 134.8722 123.0093) (end 132.1813 125.7002) (width 0.2) (layer "B.Cu") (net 1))
 (segment (start 103.8 118.8125) (end 92.075 107.0875) (width 0.2) (layer "B.Cu") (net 1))
 (segment (start 115.25 81.1875) (end 115.25 70.645) (width 0.2) (layer "B.Cu") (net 1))
 (segment (start 101.905 70.4237) (end 101.905 71.29) (width 0.2) (layer "B.Cu") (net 1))
 (segment (start 115.25 105) (end 115.25 128.8125) (width 0.2) (layer "B.Cu") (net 1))
 (segment (start 160.95 95) (end 160.95 118.8125) (width 0.2) (layer "B.Cu") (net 1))
 (segment (start 160.95 118.8125) (end 158.8088 120.9537) (width 0.2) (layer "B.Cu") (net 1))
 (segment (start 92.075 107.0875) (end 92.075 102.625) (width 0.2) (layer "B.Cu") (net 1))
 (segment (start 134.3 81.1875) (end 134.3 105) (width 0.2) (layer "B.Cu") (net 1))
 (segment (start 115.25 81.1875) (end 115.25 105) (width 0.2) (layer "B.Cu") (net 1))
 (segment (start 154.7713 120.9537) (end 148.625 127.1) (width 0.2) (layer "B.Cu") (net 1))
 (segment (start 92.075 97.375) (end 92.075 102.625) (width 0.2) (layer "B.Cu") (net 1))
 (segment (start 100.6996 69.2183) (end 101.905 70.4237) (width 0.2) (layer "B.Cu") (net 1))
 (segment (start 101.905 63.67) (end 100.6996 64.8754) (width 0.2) (layer "B.Cu") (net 1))
 (segment (start 134.0442 128.5567) (end 134.3 128.8125) (width 0.2) (layer "B.Cu") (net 1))
 (segment (start 101.905 73.83) (end 101.905 71.29) (width 0.2) (layer "B.Cu") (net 1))
 (segment (start 126.035 116.7) (end 126.035 119.554) (width 0.2) (layer "B.Cu") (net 1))
 (segment (start 115.25 70.645) (end 117.145 68.75) (width 0.2) (layer "B.Cu") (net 1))
 (segment (start 103.6402 92.9204) (end 105.9 95.1802) (width 0.2) (layer "F.Cu") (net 10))
 (segment (start 101.5674 92.9204) (end 103.6402 92.9204) (width 0.2) (layer "F.Cu") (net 10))
 (segment (start 100.7506 85.1444) (end 100.7506 92.1036) (width 0.2) (layer "F.Cu") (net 10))
 (segment (start 101.905 83.99) (end 100.7506 85.1444) (width 0.2) (layer "F.Cu") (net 10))
 (segment (start 105.9 95.1802) (end 105.9 100) (width 0.2) (layer "F.Cu") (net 10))
 (segment (start 100.7506 92.1036) (end 101.5674 92.9204) (width 0.2) (layer "F.Cu") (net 10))
 (segment (start 105.9 82.535) (end 105.9 76.1875) (width 0.2) (layer "B.Cu") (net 7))
 (segment (start 101.905 86.53) (end 105.9 82.535) (width 0.2) (layer "B.Cu") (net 7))
 (segment (start 159.7696 120.5321) (end 163.05 123.8125) (width 0.2) (layer "F.Cu") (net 11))
 (segment (start 155.2783 120.5321) (end 159.7696 120.5321) (width 0.2) (layer "F.Cu") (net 11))
 (segment (start 117.145 91.61) (end 126.3562 91.61) (width 0.2) (layer "F.Cu") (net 11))
 (segment (start 126.3562 91.61) (end 155.2783 120.5321) (width 0.2) (layer "F.Cu") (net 11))
 (segment (start 159.7696 96.7196) (end 163.05 100) (width 0.2) (layer "F.Cu") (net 4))
 (segment (start 117.145 83.99) (end 115.9758 85.1592) (width 0.2) (layer "F.Cu") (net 4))
 (segment (start 148.0636 87.7313) (end 157.0519 96.7196) (width 0.2) (layer "F.Cu") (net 4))
 (segment (start 116.6665 87.7313) (end 148.0636 87.7313) (width 0.2) (layer "F.Cu") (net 4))
 (segment (start 115.9758 87.0406) (end 116.6665 87.7313) (width 0.2) (layer "F.Cu") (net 4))
 (segment (start 157.0519 96.7196) (end 159.7696 96.7196) (width 0.2) (layer "F.Cu") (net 4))
 (segment (start 115.9758 85.1592) (end 115.9758 87.0406) (width 0.2) (layer "F.Cu") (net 4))
 (segment (start 160.7948 73.9323) (end 163.05 76.1875) (width 0.2) (layer "F.Cu") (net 12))
 (segment (start 117.145 81.45) (end 124.6627 73.9323) (width 0.2) (layer "F.Cu") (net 12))
 (segment (start 124.6627 73.9323) (end 160.7948 73.9323) (width 0.2) (layer "F.Cu") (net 12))
 (segment (start 101.905 89.07) (end 109.525 89.07) (width 0.2) (layer "F.Cu") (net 5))
 (via (at 109.525 89.07) (size 0.6) (drill 0.3) (layers "F.Cu" "B.Cu") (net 5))
 (segment (start 113.15 123.8125) (end 109.525 120.1875) (width 0.2) (layer "B.Cu") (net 5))
 (segment (start 109.525 120.1875) (end 109.525 89.07) (width 0.2) (layer "B.Cu") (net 5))
 (segment (start 104.76 91.61) (end 113.15 100) (width 0.2) (layer "F.Cu") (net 3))
 (segment (start 101.905 91.61) (end 104.76 91.61) (width 0.2) (layer "F.Cu") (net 3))
 (segment (start 113.15 83.2723) (end 113.15 76.1875) (width 0.2) (layer "B.Cu") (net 6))
 (segment (start 102.2723 94.15) (end 113.15 83.2723) (width 0.2) (layer "B.Cu") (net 6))
 (segment (start 101.905 94.15) (end 102.2723 94.15) (width 0.2) (layer "B.Cu") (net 6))
 (segment (start 117.145 94.722) (end 127.305 104.882) (width 0.2) (layer "B.Cu") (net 2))
 (segment (start 117.145 94.15) (end 117.145 94.722) (width 0.2) (layer "B.Cu") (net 2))
 (segment (start 127.305 118.9175) (end 132.2 123.8125) (width 0.2) (layer "B.Cu") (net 2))
 (segment (start 127.305 104.882) (end 127.305 118.9175) (width 0.2) (layer "B.Cu") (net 2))
 (segment (start 117.145 89.07) (end 115.9509 90.2641) (width 0.2) (layer "F.Cu") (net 13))
 (segment (start 115.9509 92.0504) (end 116.7862 92.8857) (width 0.2) (layer "F.Cu") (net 13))
 (segment (start 115.9509 90.2641) (end 115.9509 92.0504) (width 0.2) (layer "F.Cu") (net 13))
 (segment (start 125.0857 92.8857) (end 132.2 100) (width 0.2) (layer "F.Cu") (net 13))
 (segment (start 116.7862 92.8857) (end 125.0857 92.8857) (width 0.2) (layer "F.Cu") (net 13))
 (segment (start 127.4875 76.1875) (end 132.2 76.1875) (width 0.2) (layer "F.Cu") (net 8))
 (segment (start 117.145 86.53) (end 127.4875 76.1875) (width 0.2) (layer "F.Cu") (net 8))
 (segment (start 114.7996 79.5379) (end 114.7996 68.5554) (width 0.2) (layer "B.Cu") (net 14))
 (segment (start 108.775 130.0511) (end 114.4739 124.3522) (width 0.2) (layer "B.Cu") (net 14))
 (segment (start 114.7996 68.5554) (end 117.145 66.21) (width 0.2) (layer "B.Cu") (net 14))
 (segment (start 114.4739 122.1705) (end 113.8759 121.5725) (width 0.2) (layer "B.Cu") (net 14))
 (segment (start 108.775 133.765) (end 108.775 130.0511) (width 0.2) (layer "B.Cu") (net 14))
 (segment (start 114.4739 124.3522) (end 114.4739 122.1705) (width 0.2) (layer "B.Cu") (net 14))
 (segment (start 113.8759 121.5725) (end 113.8759 103.0903) (width 0.2) (layer "B.Cu") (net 14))
 (segment (start 114.4714 102.4948) (end 114.4714 99.2214) (width 0.2) (layer "B.Cu") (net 14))
 (segment (start 117.145 63.67) (end 117.145 66.21) (width 0.2) (layer "B.Cu") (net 14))
 (segment (start 113.8759 103.0903) (end 114.4714 102.4948) (width 0.2) (layer "B.Cu") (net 14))
 (segment (start 113.9251 98.6751) (end 113.9251 80.4124) (width 0.2) (layer "B.Cu") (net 14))
 (segment (start 114.4714 99.2214) (end 113.9251 98.6751) (width 0.2) (layer "B.Cu") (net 14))
 (segment (start 113.9251 80.4124) (end 114.7996 79.5379) (width 0.2) (layer "B.Cu") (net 14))
 (segment (start 117.145 71.29) (end 115.7635 72.6715) (width 0.2) (layer "F.Cu") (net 16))
 (segment (start 115.7635 72.6715) (end 93.775 72.6715) (width 0.2) (layer "F.Cu") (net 16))
 (via (at 93.775 72.6715) (size 0.6) (drill 0.3) (layers "F.Cu" "B.Cu") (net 16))
 (segment (start 93.775 97.375) (end 93.775 72.6715) (width 0.2) (layer "B.Cu") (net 16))
 (segment (start 93.775 97.375) (end 93.775 102.625) (width 0.2) (layer "B.Cu") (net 16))
 (segment (start 128.575 116.7) (end 128.575 82.4804) (width 0.2) (layer "B.Cu") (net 17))
 (segment (start 128.575 82.4804) (end 119.9246 73.83) (width 0.2) (layer "B.Cu") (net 17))
 (segment (start 119.9246 73.83) (end 117.145 73.83) (width 0.2) (layer "B.Cu") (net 17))
 (segment (start 117.27 109.3233) (end 117.27 102.2586) (width 0.2) (layer "F.Cu") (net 23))
 (segment (start 117.27 102.2586) (end 114.5876 99.5762) (width 0.2) (layer "F.Cu") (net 23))
 (segment (start 114.5876 99.5762) (end 114.5876 98.3826) (width 0.2) (layer "F.Cu") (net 23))
 (segment (start 114.5876 98.3826) (end 105.8882 89.6832) (width 0.2) (layer "F.Cu") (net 23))
 (segment (start 123.495 116.7) (end 123.495 115.5483) (width 0.2) (layer "F.Cu") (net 23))
 (segment (start 123.495 115.5483) (end 117.27 109.3233) (width 0.2) (layer "F.Cu") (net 23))
 (via (at 105.8882 89.6832) (size 0.6) (drill 0.3) (layers "F.Cu" "B.Cu") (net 23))
 (segment (start 105.8882 89.6832) (end 107.2379 88.3335) (width 0.2) (layer "B.Cu") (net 23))
 (segment (start 107.2379 71.5429) (end 101.905 66.21) (width 0.2) (layer "B.Cu") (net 23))
 (segment (start 107.2379 88.3335) (end 107.2379 71.5429) (width 0.2) (layer "B.Cu") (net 23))
 (segment (start 114.9877 91.9927) (end 114.9877 93.7099) (width 0.2) (layer "F.Cu") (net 20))
 (segment (start 118.8122 97.5344) (end 119.815 97.5344) (width 0.2) (layer "F.Cu") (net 20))
 (segment (start 114.9877 93.7099) (end 118.8122 97.5344) (width 0.2) (layer "F.Cu") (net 20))
 (segment (start 101.905 78.91) (end 114.9877 91.9927) (width 0.2) (layer "F.Cu") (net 20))
 (segment (start 131.115 108.8344) (end 131.115 116.7) (width 0.2) (layer "F.Cu") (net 20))
 (segment (start 119.815 97.5344) (end 131.115 108.8344) (width 0.2) (layer "F.Cu") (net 20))
 (segment (start 140.3658 132.4575) (end 107.275 132.4575) (width 0.2) (layer "F.Cu") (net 15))
 (segment (start 146.625 127.1) (end 145.7233 127.1) (width 0.2) (layer "F.Cu") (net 15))
 (segment (start 145.7233 127.1) (end 140.3658 132.4575) (width 0.2) (layer "F.Cu") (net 15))
 (via (at 107.275 132.4575) (size 0.6) (drill 0.3) (layers "F.Cu" "B.Cu") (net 15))
 (segment (start 107.275 133.765) (end 107.275 132.4575) (width 0.2) (layer "B.Cu") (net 15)))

